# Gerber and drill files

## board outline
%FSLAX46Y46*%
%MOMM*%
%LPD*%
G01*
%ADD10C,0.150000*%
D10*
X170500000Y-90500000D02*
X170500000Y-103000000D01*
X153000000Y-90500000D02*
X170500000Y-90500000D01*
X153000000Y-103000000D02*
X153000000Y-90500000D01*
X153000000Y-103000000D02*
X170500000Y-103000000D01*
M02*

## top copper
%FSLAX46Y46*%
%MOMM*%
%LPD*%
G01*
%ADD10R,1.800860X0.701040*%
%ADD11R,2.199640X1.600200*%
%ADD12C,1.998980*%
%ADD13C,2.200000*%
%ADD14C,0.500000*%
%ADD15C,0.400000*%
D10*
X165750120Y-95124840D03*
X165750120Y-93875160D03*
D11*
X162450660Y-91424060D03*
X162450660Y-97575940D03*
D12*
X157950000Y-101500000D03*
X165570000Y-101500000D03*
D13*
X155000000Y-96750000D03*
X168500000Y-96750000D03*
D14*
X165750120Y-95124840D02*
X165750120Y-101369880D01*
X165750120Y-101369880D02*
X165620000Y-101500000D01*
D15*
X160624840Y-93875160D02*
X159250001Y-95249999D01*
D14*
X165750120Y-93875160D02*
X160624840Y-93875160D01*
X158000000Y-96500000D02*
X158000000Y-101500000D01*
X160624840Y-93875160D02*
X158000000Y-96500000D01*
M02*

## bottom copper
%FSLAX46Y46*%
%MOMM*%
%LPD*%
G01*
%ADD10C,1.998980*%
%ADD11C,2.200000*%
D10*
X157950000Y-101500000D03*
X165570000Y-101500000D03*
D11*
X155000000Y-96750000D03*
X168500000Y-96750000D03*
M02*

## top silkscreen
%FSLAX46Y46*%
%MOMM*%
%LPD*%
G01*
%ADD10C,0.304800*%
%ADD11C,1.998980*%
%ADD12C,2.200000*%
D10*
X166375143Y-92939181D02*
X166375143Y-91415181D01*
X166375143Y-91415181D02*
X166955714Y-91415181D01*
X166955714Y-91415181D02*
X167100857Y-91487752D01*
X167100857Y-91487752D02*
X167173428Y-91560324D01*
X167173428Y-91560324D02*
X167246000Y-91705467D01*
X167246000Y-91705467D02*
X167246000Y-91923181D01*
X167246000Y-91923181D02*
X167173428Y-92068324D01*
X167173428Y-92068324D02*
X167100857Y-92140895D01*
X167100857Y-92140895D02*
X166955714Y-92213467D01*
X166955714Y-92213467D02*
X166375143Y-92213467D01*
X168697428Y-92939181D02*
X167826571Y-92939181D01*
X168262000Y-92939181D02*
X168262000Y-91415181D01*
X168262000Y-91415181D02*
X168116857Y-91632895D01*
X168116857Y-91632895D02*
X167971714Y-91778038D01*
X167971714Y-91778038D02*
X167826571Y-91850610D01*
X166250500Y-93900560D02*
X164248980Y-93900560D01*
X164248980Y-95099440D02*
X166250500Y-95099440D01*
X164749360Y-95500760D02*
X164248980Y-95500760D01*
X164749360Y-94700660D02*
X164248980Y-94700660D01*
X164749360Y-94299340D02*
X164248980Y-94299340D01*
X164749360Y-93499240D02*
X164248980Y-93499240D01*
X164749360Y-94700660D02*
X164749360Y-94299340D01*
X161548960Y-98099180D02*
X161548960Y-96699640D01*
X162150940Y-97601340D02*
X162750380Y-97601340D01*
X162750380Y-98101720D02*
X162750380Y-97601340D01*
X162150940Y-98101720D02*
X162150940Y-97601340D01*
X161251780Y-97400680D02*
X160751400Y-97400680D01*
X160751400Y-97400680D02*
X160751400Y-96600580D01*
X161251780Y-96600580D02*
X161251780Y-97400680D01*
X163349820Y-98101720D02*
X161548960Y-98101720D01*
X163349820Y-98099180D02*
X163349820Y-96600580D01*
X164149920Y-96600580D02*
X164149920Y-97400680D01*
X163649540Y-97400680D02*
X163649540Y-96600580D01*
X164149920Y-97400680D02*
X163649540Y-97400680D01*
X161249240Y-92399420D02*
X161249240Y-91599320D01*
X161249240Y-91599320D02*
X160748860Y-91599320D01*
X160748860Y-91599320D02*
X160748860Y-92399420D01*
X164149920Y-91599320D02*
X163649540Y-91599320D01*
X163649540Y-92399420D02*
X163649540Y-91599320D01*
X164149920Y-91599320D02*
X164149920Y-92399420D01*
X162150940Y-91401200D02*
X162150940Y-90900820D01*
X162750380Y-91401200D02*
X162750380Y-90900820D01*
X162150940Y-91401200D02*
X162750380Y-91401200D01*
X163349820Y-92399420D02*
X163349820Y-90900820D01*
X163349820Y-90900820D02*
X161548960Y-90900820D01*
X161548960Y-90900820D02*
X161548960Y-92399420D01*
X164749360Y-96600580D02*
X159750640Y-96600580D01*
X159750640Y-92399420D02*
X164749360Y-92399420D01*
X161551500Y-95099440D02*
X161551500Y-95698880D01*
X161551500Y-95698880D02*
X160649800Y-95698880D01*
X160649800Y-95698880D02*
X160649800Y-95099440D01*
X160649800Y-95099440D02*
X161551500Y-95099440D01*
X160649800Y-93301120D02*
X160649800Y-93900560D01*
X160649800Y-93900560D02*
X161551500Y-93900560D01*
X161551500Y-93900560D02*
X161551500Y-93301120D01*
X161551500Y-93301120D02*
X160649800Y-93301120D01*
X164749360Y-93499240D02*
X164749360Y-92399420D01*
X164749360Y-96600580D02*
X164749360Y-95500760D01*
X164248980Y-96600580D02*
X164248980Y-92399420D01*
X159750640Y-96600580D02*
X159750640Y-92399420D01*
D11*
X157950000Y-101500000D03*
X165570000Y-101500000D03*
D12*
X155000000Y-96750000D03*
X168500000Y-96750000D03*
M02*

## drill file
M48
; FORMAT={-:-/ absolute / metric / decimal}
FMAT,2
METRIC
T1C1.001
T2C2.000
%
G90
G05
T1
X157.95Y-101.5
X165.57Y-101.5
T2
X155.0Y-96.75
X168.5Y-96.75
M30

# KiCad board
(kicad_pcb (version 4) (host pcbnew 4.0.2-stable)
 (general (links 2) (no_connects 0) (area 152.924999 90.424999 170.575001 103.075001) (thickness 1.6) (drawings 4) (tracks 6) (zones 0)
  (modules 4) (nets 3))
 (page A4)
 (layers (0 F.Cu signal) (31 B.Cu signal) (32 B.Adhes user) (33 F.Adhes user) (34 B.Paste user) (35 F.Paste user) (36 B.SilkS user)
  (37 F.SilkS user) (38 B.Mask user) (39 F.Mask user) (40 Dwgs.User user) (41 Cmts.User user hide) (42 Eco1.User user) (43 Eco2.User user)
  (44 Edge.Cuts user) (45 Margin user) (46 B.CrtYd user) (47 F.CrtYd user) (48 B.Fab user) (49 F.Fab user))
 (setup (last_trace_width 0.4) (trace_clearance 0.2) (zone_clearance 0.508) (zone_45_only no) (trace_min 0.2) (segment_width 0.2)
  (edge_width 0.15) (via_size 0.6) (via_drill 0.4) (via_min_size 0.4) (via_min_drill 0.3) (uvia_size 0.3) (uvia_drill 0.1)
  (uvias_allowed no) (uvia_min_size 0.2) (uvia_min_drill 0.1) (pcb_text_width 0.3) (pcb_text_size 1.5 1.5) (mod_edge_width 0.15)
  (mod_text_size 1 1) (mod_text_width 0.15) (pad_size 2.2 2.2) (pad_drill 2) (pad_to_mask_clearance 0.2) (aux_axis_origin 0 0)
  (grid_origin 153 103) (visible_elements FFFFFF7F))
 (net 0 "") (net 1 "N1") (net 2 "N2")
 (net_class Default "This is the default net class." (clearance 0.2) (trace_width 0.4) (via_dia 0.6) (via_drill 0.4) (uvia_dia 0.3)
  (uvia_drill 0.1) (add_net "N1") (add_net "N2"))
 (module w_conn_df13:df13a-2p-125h (layer F.Cu) (at 162.25 94.5 270)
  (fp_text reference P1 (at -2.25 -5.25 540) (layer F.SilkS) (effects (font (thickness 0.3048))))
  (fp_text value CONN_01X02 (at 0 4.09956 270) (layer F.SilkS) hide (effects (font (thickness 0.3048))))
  (fp_line (start -0.59944 -4.0005) (end -0.59944 -1.99898) (layer F.SilkS) (width 0.3048))
  (fp_line (start 0.59944 -1.99898) (end 0.59944 -4.0005) (layer F.SilkS) (width 0.3048))
  (fp_line (start 1.00076 -2.49936) (end 1.00076 -1.99898) (layer F.SilkS) (width 0.3048))
  (fp_line (start 0.20066 -2.49936) (end 0.20066 -1.99898) (layer F.SilkS) (width 0.3048))
  (fp_line (start -0.20066 -2.49936) (end -0.20066 -1.99898) (layer F.SilkS) (width 0.3048))
  (fp_line (start -1.00076 -2.49936) (end -1.00076 -1.99898) (layer F.SilkS) (width 0.3048))
  (fp_line (start 0.20066 -2.49936) (end -0.20066 -2.49936) (layer F.SilkS) (width 0.3048))
  (fp_line (start 3.59918 0.70104) (end 2.19964 0.70104) (layer F.SilkS) (width 0.3048))
  (fp_line (start 3.10134 0.09906) (end 3.10134 -0.50038) (layer F.SilkS) (width 0.3048))
  (fp_line (start 3.60172 -0.50038) (end 3.10134 -0.50038) (layer F.SilkS) (width 0.3048))
  (fp_line (start 3.60172 0.09906) (end 3.10134 0.09906) (layer F.SilkS) (width 0.3048))
  (fp_line (start 2.90068 0.99822) (end 2.90068 1.4986) (layer F.SilkS) (width 0.3048))
  (fp_line (start 2.90068 1.4986) (end 2.10058 1.4986) (layer F.SilkS) (width 0.3048))
  (fp_line (start 2.10058 0.99822) (end 2.90068 0.99822) (layer F.SilkS) (width 0.3048))
  (fp_line (start 3.60172 -1.09982) (end 3.60172 0.70104) (layer F.SilkS) (width 0.3048))
  (fp_line (start 3.59918 -1.09982) (end 2.10058 -1.09982) (layer F.SilkS) (width 0.3048))
  (fp_line (start 2.10058 -1.89992) (end 2.90068 -1.89992) (layer F.SilkS) (width 0.3048))
  (fp_line (start 2.90068 -1.39954) (end 2.10058 -1.39954) (layer F.SilkS) (width 0.3048))
  (fp_line (start 2.90068 -1.89992) (end 2.90068 -1.39954) (layer F.SilkS) (width 0.3048))
  (fp_line (start -2.10058 1.00076) (end -2.90068 1.00076) (layer F.SilkS) (width 0.3048))
  (fp_line (start -2.90068 1.00076) (end -2.90068 1.50114) (layer F.SilkS) (width 0.3048))
  (fp_line (start -2.90068 1.50114) (end -2.10058 1.50114) (layer F.SilkS) (width 0.3048))
  (fp_line (start -2.90068 -1.89992) (end -2.90068 -1.39954) (layer F.SilkS) (width 0.3048))
  (fp_line (start -2.10058 -1.39954) (end -2.90068 -1.39954) (layer F.SilkS) (width 0.3048))
  (fp_line (start -2.90068 -1.89992) (end -2.10058 -1.89992) (layer F.SilkS) (width 0.3048))
  (fp_line (start -3.0988 0.09906) (end -3.59918 0.09906) (layer F.SilkS) (width 0.3048))
  (fp_line (start -3.0988 -0.50038) (end -3.59918 -0.50038) (layer F.SilkS) (width 0.3048))
  (fp_line (start -3.0988 0.09906) (end -3.0988 -0.50038) (layer F.SilkS) (width 0.3048))
  (fp_line (start -2.10058 -1.09982) (end -3.59918 -1.09982) (layer F.SilkS) (width 0.3048))
  (fp_line (start -3.59918 -1.09982) (end -3.59918 0.70104) (layer F.SilkS) (width 0.3048))
  (fp_line (start -3.59918 0.70104) (end -2.10058 0.70104) (layer F.SilkS) (width 0.3048))
  (fp_line (start 2.10058 -2.49936) (end 2.10058 2.49936) (layer F.SilkS) (width 0.3048))
  (fp_line (start -2.10058 2.49936) (end -2.10058 -2.49936) (layer F.SilkS) (width 0.3048))
  (fp_line (start 0.59944 0.6985) (end 1.19888 0.6985) (layer F.SilkS) (width 0.3048))
  (fp_line (start 1.19888 0.6985) (end 1.19888 1.6002) (layer F.SilkS) (width 0.3048))
  (fp_line (start 1.19888 1.6002) (end 0.59944 1.6002) (layer F.SilkS) (width 0.3048))
  (fp_line (start 0.59944 1.6002) (end 0.59944 0.6985) (layer F.SilkS) (width 0.3048))
  (fp_line (start -1.19888 1.6002) (end -0.59944 1.6002) (layer F.SilkS) (width 0.3048))
  (fp_line (start -0.59944 1.6002) (end -0.59944 0.6985) (layer F.SilkS) (width 0.3048))
  (fp_line (start -0.59944 0.6985) (end -1.19888 0.6985) (layer F.SilkS) (width 0.3048))
  (fp_line (start -1.19888 0.6985) (end -1.19888 1.6002) (layer F.SilkS) (width 0.3048))
  (fp_line (start -1.00076 -2.49936) (end -2.10058 -2.49936) (layer F.SilkS) (width 0.3048))
  (fp_line (start 2.10058 -2.49936) (end 1.00076 -2.49936) (layer F.SilkS) (width 0.3048))
  (fp_line (start 2.10058 -1.99898) (end -2.10058 -1.99898) (layer F.SilkS) (width 0.3048))
  (fp_line (start 2.10058 2.49936) (end -2.10058 2.49936) (layer F.SilkS) (width 0.3048))
  (pad 1 smd rect (at 0.62484 -3.50012 270) (size 0.70104 1.80086) (layers F.Cu F.Paste F.Mask) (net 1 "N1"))
  (pad 2 smd rect (at -0.62484 -3.50012 270) (size 0.70104 1.80086) (layers F.Cu F.Paste F.Mask) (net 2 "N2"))
  (pad "" smd rect (at -3.07594 -0.20066 270) (size 1.6002 2.19964) (layers F.Cu F.Paste F.Mask))
  (pad "" smd rect (at 3.07594 -0.20066 270) (size 1.6002 2.19964) (layers F.Cu F.Paste F.Mask)))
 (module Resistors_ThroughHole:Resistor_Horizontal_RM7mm (layer B.Cu) (at 157.95 101.5)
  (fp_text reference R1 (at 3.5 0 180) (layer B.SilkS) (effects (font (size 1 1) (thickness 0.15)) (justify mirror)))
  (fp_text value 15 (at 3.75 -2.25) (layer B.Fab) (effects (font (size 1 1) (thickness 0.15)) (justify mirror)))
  (pad 1 thru_hole circle (at 0 0) (size 1.99898 1.99898) (drill 1.00076) (layers *.Cu *.SilkS *.Mask) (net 2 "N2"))
  (pad 2 thru_hole circle (at 7.62 0) (size 1.99898 1.99898) (drill 1.00076) (layers *.Cu *.SilkS *.Mask) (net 1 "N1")))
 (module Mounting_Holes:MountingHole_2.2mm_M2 (layer F.Cu) (at 155 96.75) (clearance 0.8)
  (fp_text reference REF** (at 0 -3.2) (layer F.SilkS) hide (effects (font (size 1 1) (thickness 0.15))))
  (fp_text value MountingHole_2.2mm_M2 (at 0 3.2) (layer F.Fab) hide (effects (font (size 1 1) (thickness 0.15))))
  (pad "" np_thru_hole circle (at 0 0) (size 2.2 2.2) (drill 2) (layers *.Cu *.Mask F.SilkS)))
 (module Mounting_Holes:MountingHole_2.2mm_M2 (layer F.Cu) (at 168.5 96.75 90) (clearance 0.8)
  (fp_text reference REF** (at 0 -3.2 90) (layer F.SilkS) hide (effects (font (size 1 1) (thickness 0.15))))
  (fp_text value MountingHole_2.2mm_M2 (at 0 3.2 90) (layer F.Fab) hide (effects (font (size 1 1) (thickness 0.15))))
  (pad "" np_thru_hole circle (at 0 0 90) (size 2.2 2.2) (drill 2) (layers *.Cu *.Mask F.SilkS)))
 (gr_line (start 170.5 90.5) (end 170.5 103) (angle 90) (layer Edge.Cuts) (width 0.15))
 (gr_line (start 153 90.5) (end 170.5 90.5) (angle 90) (layer Edge.Cuts) (width 0.15))
 (gr_line (start 153 103) (end 153 90.5) (angle 90) (layer Edge.Cuts) (width 0.15))
 (gr_line (start 153 103) (end 170.5 103) (angle 90) (layer Edge.Cuts) (width 0.15))
 (segment (start 165.75012 95.12484) (end 165.75012 101.36988) (width 0.5) (layer F.Cu) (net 1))
 (segment (start 165.75012 101.36988) (end 165.62 101.5) (width 0.5) (layer F.Cu) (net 1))
 (segment (start 160.62484 93.87516) (end 159.250001 95.249999) (width 0.4) (layer F.Cu) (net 2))
 (segment (start 165.75012 93.87516) (end 160.62484 93.87516) (width 0.5) (layer F.Cu) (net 2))
 (segment (start 158 96.5) (end 158 101.5) (width 0.5) (layer F.Cu) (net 2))
 (segment (start 160.62484 93.87516) (end 158 96.5) (width 0.5) (layer F.Cu) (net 2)))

